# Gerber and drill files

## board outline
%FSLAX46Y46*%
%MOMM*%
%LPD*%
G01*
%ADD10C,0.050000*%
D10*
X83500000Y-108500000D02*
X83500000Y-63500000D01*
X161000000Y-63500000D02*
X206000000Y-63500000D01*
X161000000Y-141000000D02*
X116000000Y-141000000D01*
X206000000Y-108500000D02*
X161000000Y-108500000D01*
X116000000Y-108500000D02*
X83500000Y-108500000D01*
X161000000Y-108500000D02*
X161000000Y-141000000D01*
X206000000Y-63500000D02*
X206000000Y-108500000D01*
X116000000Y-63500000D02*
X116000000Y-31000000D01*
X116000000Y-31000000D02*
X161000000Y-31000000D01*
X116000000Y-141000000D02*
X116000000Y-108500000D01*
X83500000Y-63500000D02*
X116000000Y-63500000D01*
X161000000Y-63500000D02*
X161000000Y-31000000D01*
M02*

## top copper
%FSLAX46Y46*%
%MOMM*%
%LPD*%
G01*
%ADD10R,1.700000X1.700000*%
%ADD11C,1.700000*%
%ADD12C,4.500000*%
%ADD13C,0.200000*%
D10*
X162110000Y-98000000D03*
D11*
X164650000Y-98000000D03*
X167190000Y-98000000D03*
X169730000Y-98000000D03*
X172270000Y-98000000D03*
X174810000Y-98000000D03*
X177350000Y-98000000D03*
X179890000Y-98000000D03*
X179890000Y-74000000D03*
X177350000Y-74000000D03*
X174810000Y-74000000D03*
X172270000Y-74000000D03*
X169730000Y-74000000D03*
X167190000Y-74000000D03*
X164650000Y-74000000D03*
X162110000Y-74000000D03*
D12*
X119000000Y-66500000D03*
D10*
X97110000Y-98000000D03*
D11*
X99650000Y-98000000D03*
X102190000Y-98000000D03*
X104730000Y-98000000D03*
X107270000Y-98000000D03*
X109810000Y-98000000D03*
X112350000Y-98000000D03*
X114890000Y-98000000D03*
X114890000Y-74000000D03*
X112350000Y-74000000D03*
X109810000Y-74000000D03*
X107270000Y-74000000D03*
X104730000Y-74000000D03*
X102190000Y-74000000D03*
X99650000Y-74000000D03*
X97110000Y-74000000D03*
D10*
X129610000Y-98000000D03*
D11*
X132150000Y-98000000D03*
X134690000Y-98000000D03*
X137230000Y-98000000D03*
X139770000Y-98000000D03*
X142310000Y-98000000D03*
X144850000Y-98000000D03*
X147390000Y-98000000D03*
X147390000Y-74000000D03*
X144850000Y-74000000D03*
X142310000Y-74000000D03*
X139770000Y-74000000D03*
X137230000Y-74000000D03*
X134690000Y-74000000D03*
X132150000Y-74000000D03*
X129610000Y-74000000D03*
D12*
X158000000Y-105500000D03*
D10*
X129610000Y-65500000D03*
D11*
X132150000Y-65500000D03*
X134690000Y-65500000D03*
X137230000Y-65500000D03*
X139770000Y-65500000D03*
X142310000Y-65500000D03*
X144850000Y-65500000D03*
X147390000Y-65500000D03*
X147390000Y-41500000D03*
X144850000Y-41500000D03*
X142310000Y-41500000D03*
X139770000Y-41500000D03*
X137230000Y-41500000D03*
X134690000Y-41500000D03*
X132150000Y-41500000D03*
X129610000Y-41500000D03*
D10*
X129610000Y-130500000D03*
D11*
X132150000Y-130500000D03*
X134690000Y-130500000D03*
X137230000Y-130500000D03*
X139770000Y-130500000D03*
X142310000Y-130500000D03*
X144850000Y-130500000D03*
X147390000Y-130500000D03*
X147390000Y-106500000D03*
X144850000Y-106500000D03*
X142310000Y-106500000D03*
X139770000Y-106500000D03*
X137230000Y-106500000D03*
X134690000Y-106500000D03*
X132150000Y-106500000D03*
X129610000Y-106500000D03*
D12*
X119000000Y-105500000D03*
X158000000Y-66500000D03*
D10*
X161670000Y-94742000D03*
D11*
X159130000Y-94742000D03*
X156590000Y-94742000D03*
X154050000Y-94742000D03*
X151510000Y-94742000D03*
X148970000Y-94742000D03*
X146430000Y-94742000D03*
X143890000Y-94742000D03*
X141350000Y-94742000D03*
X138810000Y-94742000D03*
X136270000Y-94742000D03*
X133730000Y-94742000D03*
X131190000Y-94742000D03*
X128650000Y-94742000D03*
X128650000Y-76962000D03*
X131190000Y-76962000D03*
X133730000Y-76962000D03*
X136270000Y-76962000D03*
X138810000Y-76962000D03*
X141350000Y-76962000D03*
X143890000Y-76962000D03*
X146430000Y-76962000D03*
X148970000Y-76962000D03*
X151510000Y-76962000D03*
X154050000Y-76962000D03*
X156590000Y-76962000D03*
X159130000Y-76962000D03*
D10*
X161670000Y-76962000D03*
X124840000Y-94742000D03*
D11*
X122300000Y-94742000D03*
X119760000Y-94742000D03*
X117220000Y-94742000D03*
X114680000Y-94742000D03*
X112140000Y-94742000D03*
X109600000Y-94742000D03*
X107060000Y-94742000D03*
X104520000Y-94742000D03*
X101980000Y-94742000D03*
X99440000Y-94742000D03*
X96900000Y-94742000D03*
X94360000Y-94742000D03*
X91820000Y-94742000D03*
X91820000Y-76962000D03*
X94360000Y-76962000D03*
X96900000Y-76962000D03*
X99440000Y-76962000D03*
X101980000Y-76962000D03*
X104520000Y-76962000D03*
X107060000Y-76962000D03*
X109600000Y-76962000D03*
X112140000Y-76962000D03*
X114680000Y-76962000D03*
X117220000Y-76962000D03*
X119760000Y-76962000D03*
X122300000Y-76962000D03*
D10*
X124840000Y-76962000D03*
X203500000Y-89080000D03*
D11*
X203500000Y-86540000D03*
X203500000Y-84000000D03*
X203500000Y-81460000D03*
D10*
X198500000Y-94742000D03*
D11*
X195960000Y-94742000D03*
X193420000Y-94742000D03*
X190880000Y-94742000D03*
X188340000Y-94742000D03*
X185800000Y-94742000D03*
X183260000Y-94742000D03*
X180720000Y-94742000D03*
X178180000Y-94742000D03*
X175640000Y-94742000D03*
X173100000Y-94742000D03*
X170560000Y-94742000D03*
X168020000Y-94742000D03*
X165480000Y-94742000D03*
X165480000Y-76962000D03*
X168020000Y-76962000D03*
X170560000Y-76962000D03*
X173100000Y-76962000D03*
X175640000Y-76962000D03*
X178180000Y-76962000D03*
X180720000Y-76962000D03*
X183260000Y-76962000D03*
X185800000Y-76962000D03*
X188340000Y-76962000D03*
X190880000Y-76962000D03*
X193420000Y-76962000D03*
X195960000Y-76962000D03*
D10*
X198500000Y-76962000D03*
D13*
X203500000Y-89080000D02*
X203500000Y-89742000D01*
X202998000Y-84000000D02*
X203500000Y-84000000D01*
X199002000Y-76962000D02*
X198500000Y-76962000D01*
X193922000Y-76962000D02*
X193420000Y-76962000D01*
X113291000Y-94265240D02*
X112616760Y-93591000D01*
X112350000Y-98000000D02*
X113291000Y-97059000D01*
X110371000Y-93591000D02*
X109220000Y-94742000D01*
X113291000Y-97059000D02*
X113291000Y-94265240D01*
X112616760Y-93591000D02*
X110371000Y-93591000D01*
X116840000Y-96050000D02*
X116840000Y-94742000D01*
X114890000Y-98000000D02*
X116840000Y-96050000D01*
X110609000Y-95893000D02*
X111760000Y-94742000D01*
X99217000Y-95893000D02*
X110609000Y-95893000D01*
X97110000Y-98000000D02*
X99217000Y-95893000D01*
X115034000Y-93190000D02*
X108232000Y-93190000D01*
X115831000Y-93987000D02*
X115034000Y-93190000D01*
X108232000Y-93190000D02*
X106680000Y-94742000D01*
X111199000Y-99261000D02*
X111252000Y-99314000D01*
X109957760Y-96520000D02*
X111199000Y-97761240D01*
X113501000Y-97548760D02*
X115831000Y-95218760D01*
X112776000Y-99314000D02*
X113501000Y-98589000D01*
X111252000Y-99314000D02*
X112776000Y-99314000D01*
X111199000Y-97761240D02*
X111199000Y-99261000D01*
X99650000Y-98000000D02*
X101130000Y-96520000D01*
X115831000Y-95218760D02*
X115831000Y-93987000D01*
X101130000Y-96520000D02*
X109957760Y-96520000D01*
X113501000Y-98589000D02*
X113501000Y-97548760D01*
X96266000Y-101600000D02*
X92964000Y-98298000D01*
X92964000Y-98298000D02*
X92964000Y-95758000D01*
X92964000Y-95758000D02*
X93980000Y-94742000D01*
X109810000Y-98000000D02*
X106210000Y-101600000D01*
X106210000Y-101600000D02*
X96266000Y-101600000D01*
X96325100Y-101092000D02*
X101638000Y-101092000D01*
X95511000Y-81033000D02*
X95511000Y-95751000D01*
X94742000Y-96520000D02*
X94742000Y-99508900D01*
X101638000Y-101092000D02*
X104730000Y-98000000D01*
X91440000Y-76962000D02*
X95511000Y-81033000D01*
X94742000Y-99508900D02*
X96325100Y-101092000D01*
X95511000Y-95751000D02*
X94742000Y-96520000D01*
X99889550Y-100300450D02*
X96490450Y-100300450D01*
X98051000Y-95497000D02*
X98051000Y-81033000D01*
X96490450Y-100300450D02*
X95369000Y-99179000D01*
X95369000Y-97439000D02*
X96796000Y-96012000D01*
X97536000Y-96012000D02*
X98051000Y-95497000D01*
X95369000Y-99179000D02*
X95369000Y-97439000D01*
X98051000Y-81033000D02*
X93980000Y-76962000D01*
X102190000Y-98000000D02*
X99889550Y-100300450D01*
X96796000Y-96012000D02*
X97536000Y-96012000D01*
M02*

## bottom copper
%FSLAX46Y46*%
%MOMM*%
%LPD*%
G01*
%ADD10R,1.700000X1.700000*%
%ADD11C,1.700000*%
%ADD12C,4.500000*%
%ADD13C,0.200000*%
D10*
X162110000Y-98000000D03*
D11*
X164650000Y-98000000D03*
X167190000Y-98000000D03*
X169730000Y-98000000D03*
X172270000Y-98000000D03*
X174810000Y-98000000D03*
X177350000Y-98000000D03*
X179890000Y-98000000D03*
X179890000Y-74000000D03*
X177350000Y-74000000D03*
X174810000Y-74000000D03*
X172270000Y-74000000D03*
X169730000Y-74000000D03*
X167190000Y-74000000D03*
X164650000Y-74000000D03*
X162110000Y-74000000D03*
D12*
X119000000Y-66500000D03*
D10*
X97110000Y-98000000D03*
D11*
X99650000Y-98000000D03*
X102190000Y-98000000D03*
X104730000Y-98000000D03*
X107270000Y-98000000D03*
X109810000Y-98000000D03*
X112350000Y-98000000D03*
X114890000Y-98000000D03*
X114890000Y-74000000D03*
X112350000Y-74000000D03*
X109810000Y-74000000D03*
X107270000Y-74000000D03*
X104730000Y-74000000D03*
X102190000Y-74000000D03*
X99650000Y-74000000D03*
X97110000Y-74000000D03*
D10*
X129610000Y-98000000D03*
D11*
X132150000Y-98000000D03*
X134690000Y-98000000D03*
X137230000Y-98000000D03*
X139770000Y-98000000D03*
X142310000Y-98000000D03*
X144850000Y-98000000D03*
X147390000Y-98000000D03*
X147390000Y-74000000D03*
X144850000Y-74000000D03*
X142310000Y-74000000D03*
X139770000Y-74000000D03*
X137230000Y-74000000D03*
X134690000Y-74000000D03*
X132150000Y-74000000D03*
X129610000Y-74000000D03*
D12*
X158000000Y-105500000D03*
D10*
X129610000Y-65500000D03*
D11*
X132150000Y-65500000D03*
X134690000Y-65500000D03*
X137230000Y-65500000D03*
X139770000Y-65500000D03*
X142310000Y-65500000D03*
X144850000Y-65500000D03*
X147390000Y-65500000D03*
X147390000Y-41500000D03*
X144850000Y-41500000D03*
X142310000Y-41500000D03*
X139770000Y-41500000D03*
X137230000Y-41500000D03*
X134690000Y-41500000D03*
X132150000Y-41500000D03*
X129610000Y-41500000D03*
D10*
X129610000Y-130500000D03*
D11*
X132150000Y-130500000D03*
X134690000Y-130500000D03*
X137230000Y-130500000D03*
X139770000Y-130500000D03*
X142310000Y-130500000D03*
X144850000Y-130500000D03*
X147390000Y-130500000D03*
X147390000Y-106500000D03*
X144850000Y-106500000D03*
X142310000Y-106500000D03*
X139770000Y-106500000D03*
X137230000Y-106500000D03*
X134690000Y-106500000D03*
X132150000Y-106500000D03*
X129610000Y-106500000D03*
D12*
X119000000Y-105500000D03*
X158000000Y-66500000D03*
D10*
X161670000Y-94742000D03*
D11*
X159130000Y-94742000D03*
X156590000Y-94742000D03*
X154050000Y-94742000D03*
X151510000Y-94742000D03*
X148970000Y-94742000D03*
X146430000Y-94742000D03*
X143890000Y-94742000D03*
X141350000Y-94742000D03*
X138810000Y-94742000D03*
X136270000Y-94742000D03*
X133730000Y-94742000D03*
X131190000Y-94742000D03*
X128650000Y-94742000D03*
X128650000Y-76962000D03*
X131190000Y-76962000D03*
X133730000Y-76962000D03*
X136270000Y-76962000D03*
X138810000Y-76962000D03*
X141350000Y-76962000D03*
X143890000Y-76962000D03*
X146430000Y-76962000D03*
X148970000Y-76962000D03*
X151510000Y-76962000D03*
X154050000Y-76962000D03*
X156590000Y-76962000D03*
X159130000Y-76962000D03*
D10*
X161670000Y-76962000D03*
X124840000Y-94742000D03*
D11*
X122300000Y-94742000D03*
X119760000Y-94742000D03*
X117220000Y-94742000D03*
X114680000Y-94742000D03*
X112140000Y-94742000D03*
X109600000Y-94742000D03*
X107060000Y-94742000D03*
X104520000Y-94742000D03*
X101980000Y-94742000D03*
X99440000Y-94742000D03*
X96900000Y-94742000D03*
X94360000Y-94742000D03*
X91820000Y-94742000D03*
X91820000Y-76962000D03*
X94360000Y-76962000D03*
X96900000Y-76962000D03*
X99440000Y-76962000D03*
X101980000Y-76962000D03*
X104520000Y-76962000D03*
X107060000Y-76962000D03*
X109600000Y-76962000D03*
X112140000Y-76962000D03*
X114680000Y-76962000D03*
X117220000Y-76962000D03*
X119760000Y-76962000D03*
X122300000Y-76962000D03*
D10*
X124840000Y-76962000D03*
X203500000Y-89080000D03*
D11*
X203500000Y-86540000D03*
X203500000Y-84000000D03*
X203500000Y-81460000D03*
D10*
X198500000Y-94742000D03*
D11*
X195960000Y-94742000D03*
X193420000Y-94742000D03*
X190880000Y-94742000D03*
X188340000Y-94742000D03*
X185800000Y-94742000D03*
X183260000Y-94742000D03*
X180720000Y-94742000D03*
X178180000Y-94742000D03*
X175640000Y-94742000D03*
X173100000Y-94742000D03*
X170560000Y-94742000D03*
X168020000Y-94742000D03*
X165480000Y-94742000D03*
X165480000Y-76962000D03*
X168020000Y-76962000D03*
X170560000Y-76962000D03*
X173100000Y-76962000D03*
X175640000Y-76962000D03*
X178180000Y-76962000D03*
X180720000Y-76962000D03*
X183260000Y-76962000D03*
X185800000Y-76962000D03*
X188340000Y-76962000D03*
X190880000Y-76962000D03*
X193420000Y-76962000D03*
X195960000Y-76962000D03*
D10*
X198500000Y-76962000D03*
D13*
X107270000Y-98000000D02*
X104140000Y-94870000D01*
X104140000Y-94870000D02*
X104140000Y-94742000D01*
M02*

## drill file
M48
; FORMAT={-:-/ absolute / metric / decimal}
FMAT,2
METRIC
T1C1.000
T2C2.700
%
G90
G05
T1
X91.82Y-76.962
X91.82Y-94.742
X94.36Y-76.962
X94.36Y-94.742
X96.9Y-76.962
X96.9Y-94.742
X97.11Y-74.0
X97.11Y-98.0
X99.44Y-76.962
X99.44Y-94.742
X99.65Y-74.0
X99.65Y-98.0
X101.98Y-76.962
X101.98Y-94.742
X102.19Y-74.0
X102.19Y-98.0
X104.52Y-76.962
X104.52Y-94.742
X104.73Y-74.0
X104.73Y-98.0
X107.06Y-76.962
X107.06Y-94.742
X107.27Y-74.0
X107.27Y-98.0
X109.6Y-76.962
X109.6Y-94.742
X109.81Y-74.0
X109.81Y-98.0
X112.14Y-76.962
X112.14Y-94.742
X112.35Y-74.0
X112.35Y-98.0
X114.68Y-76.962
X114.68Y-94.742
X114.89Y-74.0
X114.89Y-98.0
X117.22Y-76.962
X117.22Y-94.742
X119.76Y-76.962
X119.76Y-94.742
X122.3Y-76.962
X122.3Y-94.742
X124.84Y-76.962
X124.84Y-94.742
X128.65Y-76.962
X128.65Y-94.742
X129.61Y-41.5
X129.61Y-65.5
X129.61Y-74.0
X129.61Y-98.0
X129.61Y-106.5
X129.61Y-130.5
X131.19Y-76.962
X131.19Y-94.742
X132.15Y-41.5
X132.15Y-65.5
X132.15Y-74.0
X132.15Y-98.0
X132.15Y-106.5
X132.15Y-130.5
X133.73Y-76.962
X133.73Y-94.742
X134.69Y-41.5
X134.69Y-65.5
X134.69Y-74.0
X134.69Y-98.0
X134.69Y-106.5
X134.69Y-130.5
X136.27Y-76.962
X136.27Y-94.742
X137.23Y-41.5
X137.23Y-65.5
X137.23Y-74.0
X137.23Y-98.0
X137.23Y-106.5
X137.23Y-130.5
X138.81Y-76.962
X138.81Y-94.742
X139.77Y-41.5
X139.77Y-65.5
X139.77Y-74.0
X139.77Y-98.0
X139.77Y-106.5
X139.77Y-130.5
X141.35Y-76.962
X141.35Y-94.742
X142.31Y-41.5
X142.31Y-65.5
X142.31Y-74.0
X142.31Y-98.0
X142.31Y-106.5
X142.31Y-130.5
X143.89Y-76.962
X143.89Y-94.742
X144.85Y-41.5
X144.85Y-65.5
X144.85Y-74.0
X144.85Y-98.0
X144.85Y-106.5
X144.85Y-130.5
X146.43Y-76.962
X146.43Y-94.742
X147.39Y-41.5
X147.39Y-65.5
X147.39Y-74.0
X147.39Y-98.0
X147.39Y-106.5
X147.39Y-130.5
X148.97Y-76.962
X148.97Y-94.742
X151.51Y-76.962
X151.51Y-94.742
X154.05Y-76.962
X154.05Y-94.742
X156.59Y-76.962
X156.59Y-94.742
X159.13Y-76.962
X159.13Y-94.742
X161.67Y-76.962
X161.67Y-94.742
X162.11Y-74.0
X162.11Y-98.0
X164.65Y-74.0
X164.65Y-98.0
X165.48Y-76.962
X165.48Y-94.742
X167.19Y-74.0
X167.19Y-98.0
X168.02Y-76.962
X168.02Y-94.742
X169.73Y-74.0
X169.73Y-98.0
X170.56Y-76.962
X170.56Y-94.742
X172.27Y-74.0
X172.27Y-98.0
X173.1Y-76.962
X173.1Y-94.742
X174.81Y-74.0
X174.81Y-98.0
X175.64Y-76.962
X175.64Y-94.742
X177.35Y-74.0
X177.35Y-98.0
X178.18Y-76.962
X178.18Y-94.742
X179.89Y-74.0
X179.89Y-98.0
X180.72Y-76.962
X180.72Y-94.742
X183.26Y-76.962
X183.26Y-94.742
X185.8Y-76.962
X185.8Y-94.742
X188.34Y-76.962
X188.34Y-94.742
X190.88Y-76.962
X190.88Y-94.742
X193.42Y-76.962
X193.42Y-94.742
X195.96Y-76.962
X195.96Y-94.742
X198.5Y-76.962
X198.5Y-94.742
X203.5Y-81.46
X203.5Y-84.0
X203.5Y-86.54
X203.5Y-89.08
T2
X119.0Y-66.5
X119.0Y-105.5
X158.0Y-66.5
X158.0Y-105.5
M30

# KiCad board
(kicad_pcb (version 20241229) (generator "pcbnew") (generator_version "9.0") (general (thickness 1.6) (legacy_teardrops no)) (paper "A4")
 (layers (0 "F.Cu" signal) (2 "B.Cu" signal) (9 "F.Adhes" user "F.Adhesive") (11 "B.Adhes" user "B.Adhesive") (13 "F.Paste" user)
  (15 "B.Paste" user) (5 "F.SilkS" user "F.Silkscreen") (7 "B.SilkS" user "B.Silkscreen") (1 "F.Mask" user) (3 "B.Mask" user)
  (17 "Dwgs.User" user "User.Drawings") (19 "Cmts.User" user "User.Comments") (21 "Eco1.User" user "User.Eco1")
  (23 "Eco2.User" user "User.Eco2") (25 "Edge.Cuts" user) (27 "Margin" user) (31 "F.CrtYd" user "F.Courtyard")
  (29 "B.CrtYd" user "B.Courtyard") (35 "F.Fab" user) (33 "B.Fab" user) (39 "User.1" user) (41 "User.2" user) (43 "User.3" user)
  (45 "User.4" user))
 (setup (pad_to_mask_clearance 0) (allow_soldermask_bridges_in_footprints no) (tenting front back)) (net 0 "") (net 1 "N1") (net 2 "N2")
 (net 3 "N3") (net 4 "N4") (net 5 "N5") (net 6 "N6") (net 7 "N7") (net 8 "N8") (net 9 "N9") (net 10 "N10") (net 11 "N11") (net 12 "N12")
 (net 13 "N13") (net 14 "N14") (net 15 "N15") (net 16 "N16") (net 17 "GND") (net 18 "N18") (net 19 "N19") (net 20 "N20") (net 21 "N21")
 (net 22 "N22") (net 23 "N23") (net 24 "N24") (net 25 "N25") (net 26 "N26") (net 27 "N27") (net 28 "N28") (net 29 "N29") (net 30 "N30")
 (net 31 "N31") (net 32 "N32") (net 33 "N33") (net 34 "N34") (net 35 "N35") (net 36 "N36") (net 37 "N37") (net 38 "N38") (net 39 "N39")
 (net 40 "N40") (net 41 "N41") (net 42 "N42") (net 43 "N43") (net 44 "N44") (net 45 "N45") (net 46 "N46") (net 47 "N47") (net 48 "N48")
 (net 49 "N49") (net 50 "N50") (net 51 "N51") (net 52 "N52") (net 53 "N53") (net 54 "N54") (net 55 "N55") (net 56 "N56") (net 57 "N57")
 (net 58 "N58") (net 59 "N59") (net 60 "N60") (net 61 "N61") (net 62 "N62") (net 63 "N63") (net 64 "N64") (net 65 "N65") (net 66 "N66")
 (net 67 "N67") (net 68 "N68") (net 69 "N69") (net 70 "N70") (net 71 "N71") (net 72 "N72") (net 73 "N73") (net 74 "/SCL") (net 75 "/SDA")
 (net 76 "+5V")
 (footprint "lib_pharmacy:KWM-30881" (layer "F.Cu") (at 171 86)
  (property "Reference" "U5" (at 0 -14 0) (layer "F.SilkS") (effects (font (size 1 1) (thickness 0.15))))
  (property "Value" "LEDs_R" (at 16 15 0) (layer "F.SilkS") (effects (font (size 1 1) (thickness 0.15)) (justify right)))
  (pad "1" thru_hole rect (at -8.89 12 90) (size 1.7 1.7) (drill 1) (layers "*.Cu" "*.Mask") (remove_unused_layers no) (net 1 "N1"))
  (pad "2" thru_hole circle (at -6.35 12 90) (size 1.7 1.7) (drill 1) (layers "*.Cu" "*.Mask") (remove_unused_layers no) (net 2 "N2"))
  (pad "3" thru_hole circle (at -3.81 12 90) (size 1.7 1.7) (drill 1) (layers "*.Cu" "*.Mask") (remove_unused_layers no) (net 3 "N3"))
  (pad "4" thru_hole circle (at -1.27 12 90) (size 1.7 1.7) (drill 1) (layers "*.Cu" "*.Mask") (remove_unused_layers no) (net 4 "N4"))
  (pad "5" thru_hole circle (at 1.27 12 90) (size 1.7 1.7) (drill 1) (layers "*.Cu" "*.Mask") (remove_unused_layers no) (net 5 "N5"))
  (pad "6" thru_hole circle (at 3.81 12 90) (size 1.7 1.7) (drill 1) (layers "*.Cu" "*.Mask") (remove_unused_layers no) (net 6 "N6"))
  (pad "7" thru_hole circle (at 6.35 12 90) (size 1.7 1.7) (drill 1) (layers "*.Cu" "*.Mask") (remove_unused_layers no) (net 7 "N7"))
  (pad "8" thru_hole circle (at 8.89 12 90) (size 1.7 1.7) (drill 1) (layers "*.Cu" "*.Mask") (remove_unused_layers no) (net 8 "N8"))
  (pad "9" thru_hole circle (at 8.89 -12 90) (size 1.7 1.7) (drill 1) (layers "*.Cu" "*.Mask") (remove_unused_layers no) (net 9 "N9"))
  (pad "10" thru_hole circle (at 6.35 -12 90) (size 1.7 1.7) (drill 1) (layers "*.Cu" "*.Mask") (remove_unused_layers no) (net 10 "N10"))
  (pad "11" thru_hole circle (at 3.81 -12 90) (size 1.7 1.7) (drill 1) (layers "*.Cu" "*.Mask") (remove_unused_layers no) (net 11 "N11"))
  (pad "12" thru_hole circle (at 1.27 -12 90) (size 1.7 1.7) (drill 1) (layers "*.Cu" "*.Mask") (remove_unused_layers no) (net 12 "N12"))
  (pad "13" thru_hole circle (at -1.27 -12 90) (size 1.7 1.7) (drill 1) (layers "*.Cu" "*.Mask") (remove_unused_layers no) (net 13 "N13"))
  (pad "14" thru_hole circle (at -3.81 -12 90) (size 1.7 1.7) (drill 1) (layers "*.Cu" "*.Mask") (remove_unused_layers no) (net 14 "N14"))
  (pad "15" thru_hole circle (at -6.35 -12 90) (size 1.7 1.7) (drill 1) (layers "*.Cu" "*.Mask") (remove_unused_layers no) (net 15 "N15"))
  (pad "16" thru_hole circle (at -8.89 -12 90) (size 1.7 1.7) (drill 1) (layers "*.Cu" "*.Mask") (remove_unused_layers no) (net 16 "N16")))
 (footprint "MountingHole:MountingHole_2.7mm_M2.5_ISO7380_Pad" (layer "F.Cu") (at 119 66.5)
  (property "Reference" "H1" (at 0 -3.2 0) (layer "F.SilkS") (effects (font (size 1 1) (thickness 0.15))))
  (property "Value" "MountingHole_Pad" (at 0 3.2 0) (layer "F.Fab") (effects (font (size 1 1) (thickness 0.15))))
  (pad "1" thru_hole circle (at 0 0) (size 4.5 4.5) (drill 2.7) (layers "*.Cu" "*.Mask") (remove_unused_layers no) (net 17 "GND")
   (zone_connect 2)))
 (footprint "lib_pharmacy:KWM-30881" (layer "F.Cu") (at 106 86)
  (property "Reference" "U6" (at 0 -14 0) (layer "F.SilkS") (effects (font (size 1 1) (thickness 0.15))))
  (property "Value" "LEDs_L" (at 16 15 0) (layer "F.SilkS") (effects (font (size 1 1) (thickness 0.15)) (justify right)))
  (pad "1" thru_hole rect (at -8.89 12 90) (size 1.7 1.7) (drill 1) (layers "*.Cu" "*.Mask") (remove_unused_layers no) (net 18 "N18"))
  (pad "2" thru_hole circle (at -6.35 12 90) (size 1.7 1.7) (drill 1) (layers "*.Cu" "*.Mask") (remove_unused_layers no) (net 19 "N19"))
  (pad "3" thru_hole circle (at -3.81 12 90) (size 1.7 1.7) (drill 1) (layers "*.Cu" "*.Mask") (remove_unused_layers no) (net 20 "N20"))
  (pad "4" thru_hole circle (at -1.27 12 90) (size 1.7 1.7) (drill 1) (layers "*.Cu" "*.Mask") (remove_unused_layers no) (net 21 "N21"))
  (pad "5" thru_hole circle (at 1.27 12 90) (size 1.7 1.7) (drill 1) (layers "*.Cu" "*.Mask") (remove_unused_layers no) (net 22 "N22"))
  (pad "6" thru_hole circle (at 3.81 12 90) (size 1.7 1.7) (drill 1) (layers "*.Cu" "*.Mask") (remove_unused_layers no) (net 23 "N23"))
  (pad "7" thru_hole circle (at 6.35 12 90) (size 1.7 1.7) (drill 1) (layers "*.Cu" "*.Mask") (remove_unused_layers no) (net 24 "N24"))
  (pad "8" thru_hole circle (at 8.89 12 90) (size 1.7 1.7) (drill 1) (layers "*.Cu" "*.Mask") (remove_unused_layers no) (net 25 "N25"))
  (pad "9" thru_hole circle (at 8.89 -12 90) (size 1.7 1.7) (drill 1) (layers "*.Cu" "*.Mask") (remove_unused_layers no) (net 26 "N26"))
  (pad "10" thru_hole circle (at 6.35 -12 90) (size 1.7 1.7) (drill 1) (layers "*.Cu" "*.Mask") (remove_unused_layers no) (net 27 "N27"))
  (pad "11" thru_hole circle (at 3.81 -12 90) (size 1.7 1.7) (drill 1) (layers "*.Cu" "*.Mask") (remove_unused_layers no) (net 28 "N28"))
  (pad "12" thru_hole circle (at 1.27 -12 90) (size 1.7 1.7) (drill 1) (layers "*.Cu" "*.Mask") (remove_unused_layers no) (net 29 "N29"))
  (pad "13" thru_hole circle (at -1.27 -12 90) (size 1.7 1.7) (drill 1) (layers "*.Cu" "*.Mask") (remove_unused_layers no) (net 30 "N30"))
  (pad "14" thru_hole circle (at -3.81 -12 90) (size 1.7 1.7) (drill 1) (layers "*.Cu" "*.Mask") (remove_unused_layers no) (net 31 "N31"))
  (pad "15" thru_hole circle (at -6.35 -12 90) (size 1.7 1.7) (drill 1) (layers "*.Cu" "*.Mask") (remove_unused_layers no) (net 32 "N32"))
  (pad "16" thru_hole circle (at -8.89 -12 90) (size 1.7 1.7) (drill 1) (layers "*.Cu" "*.Mask") (remove_unused_layers no) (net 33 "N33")))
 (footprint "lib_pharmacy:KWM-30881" (layer "F.Cu") (at 138.5 86)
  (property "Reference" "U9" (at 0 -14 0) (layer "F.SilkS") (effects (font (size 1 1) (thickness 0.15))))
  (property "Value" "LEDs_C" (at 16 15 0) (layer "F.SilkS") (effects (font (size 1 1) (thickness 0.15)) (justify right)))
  (pad "1" thru_hole rect (at -8.89 12 90) (size 1.7 1.7) (drill 1) (layers "*.Cu" "*.Mask") (remove_unused_layers no) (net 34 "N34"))
  (pad "2" thru_hole circle (at -6.35 12 90) (size 1.7 1.7) (drill 1) (layers "*.Cu" "*.Mask") (remove_unused_layers no) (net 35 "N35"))
  (pad "3" thru_hole circle (at -3.81 12 90) (size 1.7 1.7) (drill 1) (layers "*.Cu" "*.Mask") (remove_unused_layers no) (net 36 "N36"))
  (pad "4" thru_hole circle (at -1.27 12 90) (size 1.7 1.7) (drill 1) (layers "*.Cu" "*.Mask") (remove_unused_layers no) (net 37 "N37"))
  (pad "5" thru_hole circle (at 1.27 12 90) (size 1.7 1.7) (drill 1) (layers "*.Cu" "*.Mask") (remove_unused_layers no) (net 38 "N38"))
  (pad "6" thru_hole circle (at 3.81 12 90) (size 1.7 1.7) (drill 1) (layers "*.Cu" "*.Mask") (remove_unused_layers no) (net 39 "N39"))
  (pad "7" thru_hole circle (at 6.35 12 90) (size 1.7 1.7) (drill 1) (layers "*.Cu" "*.Mask") (remove_unused_layers no) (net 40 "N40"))
  (pad "8" thru_hole circle (at 8.89 12 90) (size 1.7 1.7) (drill 1) (layers "*.Cu" "*.Mask") (remove_unused_layers no) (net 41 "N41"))
  (pad "9" thru_hole circle (at 8.89 -12 90) (size 1.7 1.7) (drill 1) (layers "*.Cu" "*.Mask") (remove_unused_layers no) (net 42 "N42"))
  (pad "10" thru_hole circle (at 6.35 -12 90) (size 1.7 1.7) (drill 1) (layers "*.Cu" "*.Mask") (remove_unused_layers no) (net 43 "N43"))
  (pad "11" thru_hole circle (at 3.81 -12 90) (size 1.7 1.7) (drill 1) (layers "*.Cu" "*.Mask") (remove_unused_layers no) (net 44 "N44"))
  (pad "12" thru_hole circle (at 1.27 -12 90) (size 1.7 1.7) (drill 1) (layers "*.Cu" "*.Mask") (remove_unused_layers no) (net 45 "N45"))
  (pad "13" thru_hole circle (at -1.27 -12 90) (size 1.7 1.7) (drill 1) (layers "*.Cu" "*.Mask") (remove_unused_layers no) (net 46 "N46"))
  (pad "14" thru_hole circle (at -3.81 -12 90) (size 1.7 1.7) (drill 1) (layers "*.Cu" "*.Mask") (remove_unused_layers no) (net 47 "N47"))
  (pad "15" thru_hole circle (at -6.35 -12 90) (size 1.7 1.7) (drill 1) (layers "*.Cu" "*.Mask") (remove_unused_layers no) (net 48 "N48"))
  (pad "16" thru_hole circle (at -8.89 -12 90) (size 1.7 1.7) (drill 1) (layers "*.Cu" "*.Mask") (remove_unused_layers no) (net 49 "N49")))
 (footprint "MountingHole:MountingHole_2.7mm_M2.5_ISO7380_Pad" (layer "F.Cu") (at 158 105.5)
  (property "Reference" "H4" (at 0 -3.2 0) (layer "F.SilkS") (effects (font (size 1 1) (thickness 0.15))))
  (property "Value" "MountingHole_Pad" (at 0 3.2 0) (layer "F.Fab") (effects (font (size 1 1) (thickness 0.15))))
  (pad "1" thru_hole circle (at 0 0) (size 4.5 4.5) (drill 2.7) (layers "*.Cu" "*.Mask") (remove_unused_layers no) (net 17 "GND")
   (zone_connect 2)))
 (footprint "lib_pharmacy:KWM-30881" (layer "F.Cu") (at 138.5 53.5)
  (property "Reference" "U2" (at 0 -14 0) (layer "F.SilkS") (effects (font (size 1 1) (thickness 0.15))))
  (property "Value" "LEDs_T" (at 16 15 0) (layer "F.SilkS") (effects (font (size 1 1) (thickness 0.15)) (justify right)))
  (pad "1" thru_hole rect (at -8.89 12 90) (size 1.7 1.7) (drill 1) (layers "*.Cu" "*.Mask") (remove_unused_layers no) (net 18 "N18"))
  (pad "2" thru_hole circle (at -6.35 12 90) (size 1.7 1.7) (drill 1) (layers "*.Cu" "*.Mask") (remove_unused_layers no) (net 19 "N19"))
  (pad "3" thru_hole circle (at -3.81 12 90) (size 1.7 1.7) (drill 1) (layers "*.Cu" "*.Mask") (remove_unused_layers no) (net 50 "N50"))
  (pad "4" thru_hole circle (at -1.27 12 90) (size 1.7 1.7) (drill 1) (layers "*.Cu" "*.Mask") (remove_unused_layers no) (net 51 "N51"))
  (pad "5" thru_hole circle (at 1.27 12 90) (size 1.7 1.7) (drill 1) (layers "*.Cu" "*.Mask") (remove_unused_layers no) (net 22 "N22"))
  (pad "6" thru_hole circle (at 3.81 12 90) (size 1.7 1.7) (drill 1) (layers "*.Cu" "*.Mask") (remove_unused_layers no) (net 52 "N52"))
  (pad "7" thru_hole circle (at 6.35 12 90) (size 1.7 1.7) (drill 1) (layers "*.Cu" "*.Mask") (remove_unused_layers no) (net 24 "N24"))
  (pad "8" thru_hole circle (at 8.89 12 90) (size 1.7 1.7) (drill 1) (layers "*.Cu" "*.Mask") (remove_unused_layers no) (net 25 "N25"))
  (pad "9" thru_hole circle (at 8.89 -12 90) (size 1.7 1.7) (drill 1) (layers "*.Cu" "*.Mask") (remove_unused_layers no) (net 26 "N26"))
  (pad "10" thru_hole circle (at 6.35 -12 90) (size 1.7 1.7) (drill 1) (layers "*.Cu" "*.Mask") (remove_unused_layers no) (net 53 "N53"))
  (pad "11" thru_hole circle (at 3.81 -12 90) (size 1.7 1.7) (drill 1) (layers "*.Cu" "*.Mask") (remove_unused_layers no) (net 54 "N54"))
  (pad "12" thru_hole circle (at 1.27 -12 90) (size 1.7 1.7) (drill 1) (layers "*.Cu" "*.Mask") (remove_unused_layers no) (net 29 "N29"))
  (pad "13" thru_hole circle (at -1.27 -12 90) (size 1.7 1.7) (drill 1) (layers "*.Cu" "*.Mask") (remove_unused_layers no) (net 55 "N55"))
  (pad "14" thru_hole circle (at -3.81 -12 90) (size 1.7 1.7) (drill 1) (layers "*.Cu" "*.Mask") (remove_unused_layers no) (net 31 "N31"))
  (pad "15" thru_hole circle (at -6.35 -12 90) (size 1.7 1.7) (drill 1) (layers "*.Cu" "*.Mask") (remove_unused_layers no) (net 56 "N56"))
  (pad "16" thru_hole circle (at -8.89 -12 90) (size 1.7 1.7) (drill 1) (layers "*.Cu" "*.Mask") (remove_unused_layers no) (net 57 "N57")))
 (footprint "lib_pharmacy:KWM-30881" (layer "F.Cu") (at 138.5 118.5)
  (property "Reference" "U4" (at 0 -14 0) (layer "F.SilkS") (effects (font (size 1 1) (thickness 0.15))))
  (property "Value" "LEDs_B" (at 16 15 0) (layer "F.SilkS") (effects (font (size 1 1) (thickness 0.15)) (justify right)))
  (pad "1" thru_hole rect (at -8.89 12 90) (size 1.7 1.7) (drill 1) (layers "*.Cu" "*.Mask") (remove_unused_layers no) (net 1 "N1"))
  (pad "2" thru_hole circle (at -6.35 12 90) (size 1.7 1.7) (drill 1) (layers "*.Cu" "*.Mask") (remove_unused_layers no) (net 2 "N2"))
  (pad "3" thru_hole circle (at -3.81 12 90) (size 1.7 1.7) (drill 1) (layers "*.Cu" "*.Mask") (remove_unused_layers no) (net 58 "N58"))
  (pad "4" thru_hole circle (at -1.27 12 90) (size 1.7 1.7) (drill 1) (layers "*.Cu" "*.Mask") (remove_unused_layers no) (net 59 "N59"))
  (pad "5" thru_hole circle (at 1.27 12 90) (size 1.7 1.7) (drill 1) (layers "*.Cu" "*.Mask") (remove_unused_layers no) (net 5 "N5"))
  (pad "6" thru_hole circle (at 3.81 12 90) (size 1.7 1.7) (drill 1) (layers "*.Cu" "*.Mask") (remove_unused_layers no) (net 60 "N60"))
  (pad "7" thru_hole circle (at 6.35 12 90) (size 1.7 1.7) (drill 1) (layers "*.Cu" "*.Mask") (remove_unused_layers no) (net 7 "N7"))
  (pad "8" thru_hole circle (at 8.89 12 90) (size 1.7 1.7) (drill 1) (layers "*.Cu" "*.Mask") (remove_unused_layers no) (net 8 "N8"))
  (pad "9" thru_hole circle (at 8.89 -12 90) (size 1.7 1.7) (drill 1) (layers "*.Cu" "*.Mask") (remove_unused_layers no) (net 9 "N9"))
  (pad "10" thru_hole circle (at 6.35 -12 90) (size 1.7 1.7) (drill 1) (layers "*.Cu" "*.Mask") (remove_unused_layers no) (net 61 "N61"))
  (pad "11" thru_hole circle (at 3.81 -12 90) (size 1.7 1.7) (drill 1) (layers "*.Cu" "*.Mask") (remove_unused_layers no) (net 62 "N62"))
  (pad "12" thru_hole circle (at 1.27 -12 90) (size 1.7 1.7) (drill 1) (layers "*.Cu" "*.Mask") (remove_unused_layers no) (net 12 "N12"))
  (pad "13" thru_hole circle (at -1.27 -12 90) (size 1.7 1.7) (drill 1) (layers "*.Cu" "*.Mask") (remove_unused_layers no) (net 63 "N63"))
  (pad "14" thru_hole circle (at -3.81 -12 90) (size 1.7 1.7) (drill 1) (layers "*.Cu" "*.Mask") (remove_unused_layers no) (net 14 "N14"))
  (pad "15" thru_hole circle (at -6.35 -12 90) (size 1.7 1.7) (drill 1) (layers "*.Cu" "*.Mask") (remove_unused_layers no) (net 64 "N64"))
  (pad "16" thru_hole circle (at -8.89 -12 90) (size 1.7 1.7) (drill 1) (layers "*.Cu" "*.Mask") (remove_unused_layers no) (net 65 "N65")))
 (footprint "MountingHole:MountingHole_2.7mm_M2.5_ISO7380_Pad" (layer "F.Cu") (at 119 105.5)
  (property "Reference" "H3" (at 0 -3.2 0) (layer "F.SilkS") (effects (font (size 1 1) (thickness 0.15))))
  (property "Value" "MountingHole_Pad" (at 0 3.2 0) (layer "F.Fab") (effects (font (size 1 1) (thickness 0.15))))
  (pad "1" thru_hole circle (at 0 0) (size 4.5 4.5) (drill 2.7) (layers "*.Cu" "*.Mask") (remove_unused_layers no) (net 17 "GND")
   (zone_connect 2)))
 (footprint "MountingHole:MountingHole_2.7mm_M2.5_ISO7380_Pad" (layer "F.Cu") (at 158 66.5)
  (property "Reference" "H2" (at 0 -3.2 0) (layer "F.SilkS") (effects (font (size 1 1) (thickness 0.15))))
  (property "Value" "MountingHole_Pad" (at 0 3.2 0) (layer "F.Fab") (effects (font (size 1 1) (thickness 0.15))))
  (pad "1" thru_hole circle (at 0 0) (size 4.5 4.5) (drill 2.7) (layers "*.Cu" "*.Mask") (remove_unused_layers no) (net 17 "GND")
   (zone_connect 2)))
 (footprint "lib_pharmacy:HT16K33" (layer "B.Cu") (at 161.67 94.742 180)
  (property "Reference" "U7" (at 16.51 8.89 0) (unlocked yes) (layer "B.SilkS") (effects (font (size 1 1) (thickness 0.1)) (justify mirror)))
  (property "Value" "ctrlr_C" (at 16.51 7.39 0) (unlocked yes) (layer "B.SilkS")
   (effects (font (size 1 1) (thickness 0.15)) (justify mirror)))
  (pad "1" thru_hole rect (at 0 0 90) (size 1.7 1.7) (drill 1) (layers "*.Cu" "*.Mask") (remove_unused_layers no) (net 17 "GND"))
  (pad "2" thru_hole circle (at 2.54 0 90) (size 1.7 1.7) (drill 1) (layers "*.Cu" "*.Mask") (remove_unused_layers no) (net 42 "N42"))
  (pad "3" thru_hole circle (at 5.08 0 90) (size 1.7 1.7) (drill 1) (layers "*.Cu" "*.Mask") (remove_unused_layers no) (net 47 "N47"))
  (pad "4" thru_hole circle (at 7.62 0 90) (size 1.7 1.7) (drill 1) (layers "*.Cu" "*.Mask") (remove_unused_layers no) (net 41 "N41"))
  (pad "5" thru_hole circle (at 10.16 0 90) (size 1.7 1.7) (drill 1) (layers "*.Cu" "*.Mask") (remove_unused_layers no) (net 45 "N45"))
  (pad "6" thru_hole circle (at 12.7 0 90) (size 1.7 1.7) (drill 1) (layers "*.Cu" "*.Mask") (remove_unused_layers no) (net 34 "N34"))
  (pad "7" thru_hole circle (at 15.24 0 90) (size 1.7 1.7) (drill 1) (layers "*.Cu" "*.Mask") (remove_unused_layers no) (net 40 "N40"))
  (pad "8" thru_hole circle (at 17.78 0 90) (size 1.7 1.7) (drill 1) (layers "*.Cu" "*.Mask") (remove_unused_layers no) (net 35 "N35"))
  (pad "9" thru_hole circle (at 20.32 0 90) (size 1.7 1.7) (drill 1) (layers "*.Cu" "*.Mask") (remove_unused_layers no) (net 38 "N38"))
  (pad "10" thru_hole circle (at 22.86 0 90) (size 1.7 1.7) (drill 1) (layers "*.Cu" "*.Mask") (remove_unused_layers no) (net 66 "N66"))
  (pad "11" thru_hole circle (at 25.4 0 90) (size 1.7 1.7) (drill 1) (layers "*.Cu" "*.Mask") (remove_unused_layers no) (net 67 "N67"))
  (pad "12" thru_hole circle (at 27.94 0 90) (size 1.7 1.7) (drill 1) (layers "*.Cu" "*.Mask") (remove_unused_layers no) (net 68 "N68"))
  (pad "13" thru_hole circle (at 30.48 0 90) (size 1.7 1.7) (drill 1) (layers "*.Cu" "*.Mask") (remove_unused_layers no) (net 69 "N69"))
  (pad "14" thru_hole circle (at 33.02 0 90) (size 1.7 1.7) (drill 1) (layers "*.Cu" "*.Mask") (remove_unused_layers no) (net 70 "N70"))
  (pad "15" thru_hole circle (at 33.02 17.78 90) (size 1.7 1.7) (drill 1) (layers "*.Cu" "*.Mask") (remove_unused_layers no) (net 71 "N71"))
  (pad "16" thru_hole circle (at 30.48 17.78 90) (size 1.7 1.7) (drill 1) (layers "*.Cu" "*.Mask") (remove_unused_layers no) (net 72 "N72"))
  (pad "17" thru_hole circle (at 27.94 17.78 90) (size 1.7 1.7) (drill 1) (layers "*.Cu" "*.Mask") (remove_unused_layers no) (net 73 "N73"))
  (pad "18" thru_hole circle (at 25.4 17.78 90) (size 1.7 1.7) (drill 1) (layers "*.Cu" "*.Mask") (remove_unused_layers no) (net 49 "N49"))
  (pad "19" thru_hole circle (at 22.86 17.78 90) (size 1.7 1.7) (drill 1) (layers "*.Cu" "*.Mask") (remove_unused_layers no) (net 48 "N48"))
  (pad "20" thru_hole circle (at 20.32 17.78 90) (size 1.7 1.7) (drill 1) (layers "*.Cu" "*.Mask") (remove_unused_layers no) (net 44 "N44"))
  (pad "21" thru_hole circle (at 17.78 17.78 90) (size 1.7 1.7) (drill 1) (layers "*.Cu" "*.Mask") (remove_unused_layers no) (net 39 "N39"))
  (pad "22" thru_hole circle (at 15.24 17.78 90) (size 1.7 1.7) (drill 1) (layers "*.Cu" "*.Mask") (remove_unused_layers no) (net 43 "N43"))
  (pad "23" thru_hole circle (at 12.7 17.78 90) (size 1.7 1.7) (drill 1) (layers "*.Cu" "*.Mask") (remove_unused_layers no) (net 37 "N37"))
  (pad "24" thru_hole circle (at 10.16 17.78 90) (size 1.7 1.7) (drill 1) (layers "*.Cu" "*.Mask") (remove_unused_layers no) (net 36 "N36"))
  (pad "25" thru_hole circle (at 7.62 17.78 90) (size 1.7 1.7) (drill 1) (layers "*.Cu" "*.Mask") (remove_unused_layers no) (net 46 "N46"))
  (pad "26" thru_hole circle (at 5.08 17.78 90) (size 1.7 1.7) (drill 1) (layers "*.Cu" "*.Mask") (remove_unused_layers no) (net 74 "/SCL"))
  (pad "27" thru_hole circle (at 2.54 17.78 90) (size 1.7 1.7) (drill 1) (layers "*.Cu" "*.Mask") (remove_unused_layers no) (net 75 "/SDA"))
  (pad "28" thru_hole rect (at 0 17.78 90) (size 1.7 1.7) (drill 1) (layers "*.Cu" "*.Mask") (remove_unused_layers no) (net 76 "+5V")))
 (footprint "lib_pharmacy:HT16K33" (layer "B.Cu") (at 124.84 94.742 180)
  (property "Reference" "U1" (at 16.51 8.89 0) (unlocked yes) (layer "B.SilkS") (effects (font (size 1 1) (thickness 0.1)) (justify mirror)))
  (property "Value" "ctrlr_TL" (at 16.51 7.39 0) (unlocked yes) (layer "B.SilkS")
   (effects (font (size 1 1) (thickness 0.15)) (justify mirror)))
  (pad "1" thru_hole rect (at 0 0 90) (size 1.7 1.7) (drill 1) (layers "*.Cu" "*.Mask") (remove_unused_layers no) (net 17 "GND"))
  (pad "2" thru_hole circle (at 2.54 0 90) (size 1.7 1.7) (drill 1) (layers "*.Cu" "*.Mask") (remove_unused_layers no) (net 26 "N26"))
  (pad "3" thru_hole circle (at 5.08 0 90) (size 1.7 1.7) (drill 1) (layers "*.Cu" "*.Mask") (remove_unused_layers no) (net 31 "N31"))
  (pad "4" thru_hole circle (at 7.62 0 90) (size 1.7 1.7) (drill 1) (layers "*.Cu" "*.Mask") (remove_unused_layers no) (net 25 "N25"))
  (pad "5" thru_hole circle (at 10.16 0 90) (size 1.7 1.7) (drill 1) (layers "*.Cu" "*.Mask") (remove_unused_layers no) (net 29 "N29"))
  (pad "6" thru_hole circle (at 12.7 0 90) (size 1.7 1.7) (drill 1) (layers "*.Cu" "*.Mask") (remove_unused_layers no) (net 18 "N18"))
  (pad "7" thru_hole circle (at 15.24 0 90) (size 1.7 1.7) (drill 1) (layers "*.Cu" "*.Mask") (remove_unused_layers no) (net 24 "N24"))
  (pad "8" thru_hole circle (at 17.78 0 90) (size 1.7 1.7) (drill 1) (layers "*.Cu" "*.Mask") (remove_unused_layers no) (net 19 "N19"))
  (pad "9" thru_hole circle (at 20.32 0 90) (size 1.7 1.7) (drill 1) (layers "*.Cu" "*.Mask") (remove_unused_layers no) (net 22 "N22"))
  (pad "10" thru_hole circle (at 22.86 0 90) (size 1.7 1.7) (drill 1) (layers "*.Cu" "*.Mask") (remove_unused_layers no) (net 33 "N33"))
  (pad "11" thru_hole circle (at 25.4 0 90) (size 1.7 1.7) (drill 1) (layers "*.Cu" "*.Mask") (remove_unused_layers no) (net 32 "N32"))
  (pad "12" thru_hole circle (at 27.94 0 90) (size 1.7 1.7) (drill 1) (layers "*.Cu" "*.Mask") (remove_unused_layers no) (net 28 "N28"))
  (pad "13" thru_hole circle (at 30.48 0 90) (size 1.7 1.7) (drill 1) (layers "*.Cu" "*.Mask") (remove_unused_layers no) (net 23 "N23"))
  (pad "14" thru_hole circle (at 33.02 0 90) (size 1.7 1.7) (drill 1) (layers "*.Cu" "*.Mask") (remove_unused_layers no) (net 27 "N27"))
  (pad "15" thru_hole circle (at 33.02 17.78 90) (size 1.7 1.7) (drill 1) (layers "*.Cu" "*.Mask") (remove_unused_layers no) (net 21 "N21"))
  (pad "16" thru_hole circle (at 30.48 17.78 90) (size 1.7 1.7) (drill 1) (layers "*.Cu" "*.Mask") (remove_unused_layers no) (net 20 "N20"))
  (pad "17" thru_hole circle (at 27.94 17.78 90) (size 1.7 1.7) (drill 1) (layers "*.Cu" "*.Mask") (remove_unused_layers no) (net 30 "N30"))
  (pad "18" thru_hole circle (at 25.4 17.78 90) (size 1.7 1.7) (drill 1) (layers "*.Cu" "*.Mask") (remove_unused_layers no) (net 57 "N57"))
  (pad "19" thru_hole circle (at 22.86 17.78 90) (size 1.7 1.7) (drill 1) (layers "*.Cu" "*.Mask") (remove_unused_layers no) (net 56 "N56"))
  (pad "20" thru_hole circle (at 20.32 17.78 90) (size 1.7 1.7) (drill 1) (layers "*.Cu" "*.Mask") (remove_unused_layers no) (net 54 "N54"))
  (pad "21" thru_hole circle (at 17.78 17.78 90) (size 1.7 1.7) (drill 1) (layers "*.Cu" "*.Mask") (remove_unused_layers no) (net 52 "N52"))
  (pad "22" thru_hole circle (at 15.24 17.78 90) (size 1.7 1.7) (drill 1) (layers "*.Cu" "*.Mask") (remove_unused_layers no) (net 53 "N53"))
  (pad "23" thru_hole circle (at 12.7 17.78 90) (size 1.7 1.7) (drill 1) (layers "*.Cu" "*.Mask") (remove_unused_layers no) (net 51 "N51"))
  (pad "24" thru_hole circle (at 10.16 17.78 90) (size 1.7 1.7) (drill 1) (layers "*.Cu" "*.Mask") (remove_unused_layers no) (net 50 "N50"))
  (pad "25" thru_hole circle (at 7.62 17.78 90) (size 1.7 1.7) (drill 1) (layers "*.Cu" "*.Mask") (remove_unused_layers no) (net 55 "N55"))
  (pad "26" thru_hole circle (at 5.08 17.78 90) (size 1.7 1.7) (drill 1) (layers "*.Cu" "*.Mask") (remove_unused_layers no) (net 74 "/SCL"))
  (pad "27" thru_hole circle (at 2.54 17.78 90) (size 1.7 1.7) (drill 1) (layers "*.Cu" "*.Mask") (remove_unused_layers no) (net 75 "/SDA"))
  (pad "28" thru_hole rect (at 0 17.78 90) (size 1.7 1.7) (drill 1) (layers "*.Cu" "*.Mask") (remove_unused_layers no) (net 76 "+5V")))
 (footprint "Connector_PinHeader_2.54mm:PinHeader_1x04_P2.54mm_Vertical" (layer "B.Cu") (at 203.5 89.08)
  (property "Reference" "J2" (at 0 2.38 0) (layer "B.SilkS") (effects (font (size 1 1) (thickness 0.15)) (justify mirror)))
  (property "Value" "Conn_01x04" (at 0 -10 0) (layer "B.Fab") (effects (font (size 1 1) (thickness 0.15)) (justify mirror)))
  (pad "1" thru_hole rect (at 0 0) (size 1.7 1.7) (drill 1) (layers "*.Cu" "*.Mask") (remove_unused_layers no) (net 17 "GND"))
  (pad "2" thru_hole circle (at 0 -2.54) (size 1.7 1.7) (drill 1) (layers "*.Cu" "*.Mask") (remove_unused_layers no) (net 74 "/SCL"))
  (pad "3" thru_hole circle (at 0 -5.08) (size 1.7 1.7) (drill 1) (layers "*.Cu" "*.Mask") (remove_unused_layers no) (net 75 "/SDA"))
  (pad "4" thru_hole circle (at 0 -7.62) (size 1.7 1.7) (drill 1) (layers "*.Cu" "*.Mask") (remove_unused_layers no) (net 76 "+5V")))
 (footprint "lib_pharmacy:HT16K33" (layer "B.Cu") (at 198.5 94.742 180)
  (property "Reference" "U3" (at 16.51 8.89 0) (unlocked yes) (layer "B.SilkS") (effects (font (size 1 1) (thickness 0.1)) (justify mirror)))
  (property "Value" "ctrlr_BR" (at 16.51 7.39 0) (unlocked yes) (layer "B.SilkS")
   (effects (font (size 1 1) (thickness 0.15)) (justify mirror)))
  (pad "1" thru_hole rect (at 0 0 90) (size 1.7 1.7) (drill 1) (layers "*.Cu" "*.Mask") (remove_unused_layers no) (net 17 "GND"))
  (pad "2" thru_hole circle (at 2.54 0 90) (size 1.7 1.7) (drill 1) (layers "*.Cu" "*.Mask") (remove_unused_layers no) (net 9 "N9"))
  (pad "3" thru_hole circle (at 5.08 0 90) (size 1.7 1.7) (drill 1) (layers "*.Cu" "*.Mask") (remove_unused_layers no) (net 14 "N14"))
  (pad "4" thru_hole circle (at 7.62 0 90) (size 1.7 1.7) (drill 1) (layers "*.Cu" "*.Mask") (remove_unused_layers no) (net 8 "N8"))
  (pad "5" thru_hole circle (at 10.16 0 90) (size 1.7 1.7) (drill 1) (layers "*.Cu" "*.Mask") (remove_unused_layers no) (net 12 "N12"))
  (pad "6" thru_hole circle (at 12.7 0 90) (size 1.7 1.7) (drill 1) (layers "*.Cu" "*.Mask") (remove_unused_layers no) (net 1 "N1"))
  (pad "7" thru_hole circle (at 15.24 0 90) (size 1.7 1.7) (drill 1) (layers "*.Cu" "*.Mask") (remove_unused_layers no) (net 7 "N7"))
  (pad "8" thru_hole circle (at 17.78 0 90) (size 1.7 1.7) (drill 1) (layers "*.Cu" "*.Mask") (remove_unused_layers no) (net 2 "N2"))
  (pad "9" thru_hole circle (at 20.32 0 90) (size 1.7 1.7) (drill 1) (layers "*.Cu" "*.Mask") (remove_unused_layers no) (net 5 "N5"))
  (pad "10" thru_hole circle (at 22.86 0 90) (size 1.7 1.7) (drill 1) (layers "*.Cu" "*.Mask") (remove_unused_layers no) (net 65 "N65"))
  (pad "11" thru_hole circle (at 25.4 0 90) (size 1.7 1.7) (drill 1) (layers "*.Cu" "*.Mask") (remove_unused_layers no) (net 64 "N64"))
  (pad "12" thru_hole circle (at 27.94 0 90) (size 1.7 1.7) (drill 1) (layers "*.Cu" "*.Mask") (remove_unused_layers no) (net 62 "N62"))
  (pad "13" thru_hole circle (at 30.48 0 90) (size 1.7 1.7) (drill 1) (layers "*.Cu" "*.Mask") (remove_unused_layers no) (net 60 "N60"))
  (pad "14" thru_hole circle (at 33.02 0 90) (size 1.7 1.7) (drill 1) (layers "*.Cu" "*.Mask") (remove_unused_layers no) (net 61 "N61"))
  (pad "15" thru_hole circle (at 33.02 17.78 90) (size 1.7 1.7) (drill 1) (layers "*.Cu" "*.Mask") (remove_unused_layers no) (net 59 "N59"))
  (pad "16" thru_hole circle (at 30.48 17.78 90) (size 1.7 1.7) (drill 1) (layers "*.Cu" "*.Mask") (remove_unused_layers no) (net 58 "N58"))
  (pad "17" thru_hole circle (at 27.94 17.78 90) (size 1.7 1.7) (drill 1) (layers "*.Cu" "*.Mask") (remove_unused_layers no) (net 63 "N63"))
  (pad "18" thru_hole circle (at 25.4 17.78 90) (size 1.7 1.7) (drill 1) (layers "*.Cu" "*.Mask") (remove_unused_layers no) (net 16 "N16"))
  (pad "19" thru_hole circle (at 22.86 17.78 90) (size 1.7 1.7) (drill 1) (layers "*.Cu" "*.Mask") (remove_unused_layers no) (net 15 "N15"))
  (pad "20" thru_hole circle (at 20.32 17.78 90) (size 1.7 1.7) (drill 1) (layers "*.Cu" "*.Mask") (remove_unused_layers no) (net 11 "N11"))
  (pad "21" thru_hole circle (at 17.78 17.78 90) (size 1.7 1.7) (drill 1) (layers "*.Cu" "*.Mask") (remove_unused_layers no) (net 6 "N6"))
  (pad "22" thru_hole circle (at 15.24 17.78 90) (size 1.7 1.7) (drill 1) (layers "*.Cu" "*.Mask") (remove_unused_layers no) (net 10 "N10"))
  (pad "23" thru_hole circle (at 12.7 17.78 90) (size 1.7 1.7) (drill 1) (layers "*.Cu" "*.Mask") (remove_unused_layers no) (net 4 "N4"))
  (pad "24" thru_hole circle (at 10.16 17.78 90) (size 1.7 1.7) (drill 1) (layers "*.Cu" "*.Mask") (remove_unused_layers no) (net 3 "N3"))
  (pad "25" thru_hole circle (at 7.62 17.78 90) (size 1.7 1.7) (drill 1) (layers "*.Cu" "*.Mask") (remove_unused_layers no) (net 13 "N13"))
  (pad "26" thru_hole circle (at 5.08 17.78 90) (size 1.7 1.7) (drill 1) (layers "*.Cu" "*.Mask") (remove_unused_layers no) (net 74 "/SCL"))
  (pad "27" thru_hole circle (at 2.54 17.78 90) (size 1.7 1.7) (drill 1) (layers "*.Cu" "*.Mask") (remove_unused_layers no) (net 75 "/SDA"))
  (pad "28" thru_hole rect (at 0 17.78 90) (size 1.7 1.7) (drill 1) (layers "*.Cu" "*.Mask") (remove_unused_layers no) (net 76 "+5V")))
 (gr_line (start 83.5 108.5) (end 83.5 63.5) (stroke (width 0.05) (type default)) (layer "Edge.Cuts"))
 (gr_line (start 161 63.5) (end 206 63.5) (stroke (width 0.05) (type default)) (layer "Edge.Cuts"))
 (gr_line (start 161 141) (end 116 141) (stroke (width 0.05) (type default)) (layer "Edge.Cuts"))
 (gr_line (start 206 108.5) (end 161 108.5) (stroke (width 0.05) (type default)) (layer "Edge.Cuts"))
 (gr_line (start 116 108.5) (end 83.5 108.5) (stroke (width 0.05) (type default)) (layer "Edge.Cuts"))
 (gr_line (start 161 108.5) (end 161 141) (stroke (width 0.05) (type default)) (layer "Edge.Cuts"))
 (gr_line (start 206 63.5) (end 206 108.5) (stroke (width 0.05) (type default)) (layer "Edge.Cuts"))
 (gr_line (start 116 63.5) (end 116 31) (stroke (width 0.05) (type default)) (layer "Edge.Cuts"))
 (gr_line (start 116 31) (end 161 31) (stroke (width 0.05) (type default)) (layer "Edge.Cuts"))
 (gr_line (start 116 141) (end 116 108.5) (stroke (width 0.05) (type default)) (layer "Edge.Cuts"))
 (gr_line (start 83.5 63.5) (end 116 63.5) (stroke (width 0.05) (type default)) (layer "Edge.Cuts"))
 (gr_line (start 161 63.5) (end 161 31) (stroke (width 0.05) (type default)) (layer "Edge.Cuts"))
 (segment (start 203.5 89.08) (end 203.5 89.742) (width 0.2) (layer "F.Cu") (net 17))
 (segment (start 202.998 84) (end 203.5 84) (width 0.2) (layer "F.Cu") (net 75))
 (segment (start 199.002 76.962) (end 198.5 76.962) (width 0.2) (layer "F.Cu") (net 76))
 (segment (start 193.922 76.962) (end 193.42 76.962) (width 0.2) (layer "F.Cu") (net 74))
 (segment (start 107.27 98) (end 104.14 94.87) (width 0.2) (layer "B.Cu") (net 22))
 (segment (start 104.14 94.87) (end 104.14 94.742) (width 0.2) (layer "B.Cu") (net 22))
 (segment (start 113.291 94.26524) (end 112.61676 93.591) (width 0.2) (layer "F.Cu") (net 24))
 (segment (start 112.35 98) (end 113.291 97.059) (width 0.2) (layer "F.Cu") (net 24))
 (segment (start 110.371 93.591) (end 109.22 94.742) (width 0.2) (layer "F.Cu") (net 24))
 (segment (start 113.291 97.059) (end 113.291 94.26524) (width 0.2) (layer "F.Cu") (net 24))
 (segment (start 112.61676 93.591) (end 110.371 93.591) (width 0.2) (layer "F.Cu") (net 24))
 (segment (start 116.84 96.05) (end 116.84 94.742) (width 0.2) (layer "F.Cu") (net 25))
 (segment (start 114.89 98) (end 116.84 96.05) (width 0.2) (layer "F.Cu") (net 25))
 (segment (start 110.609 95.893) (end 111.76 94.742) (width 0.2) (layer "F.Cu") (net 18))
 (segment (start 99.217 95.893) (end 110.609 95.893) (width 0.2) (layer "F.Cu") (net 18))
 (segment (start 97.11 98) (end 99.217 95.893) (width 0.2) (layer "F.Cu") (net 18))
 (segment (start 115.034 93.19) (end 108.232 93.19) (width 0.2) (layer "F.Cu") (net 19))
 (segment (start 115.831 93.987) (end 115.034 93.19) (width 0.2) (layer "F.Cu") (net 19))
 (segment (start 108.232 93.19) (end 106.68 94.742) (width 0.2) (layer "F.Cu") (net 19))
 (segment (start 111.199 99.261) (end 111.252 99.314) (width 0.2) (layer "F.Cu") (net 19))
 (segment (start 109.95776 96.52) (end 111.199 97.76124) (width 0.2) (layer "F.Cu") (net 19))
 (segment (start 113.501 97.54876) (end 115.831 95.21876) (width 0.2) (layer "F.Cu") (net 19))
 (segment (start 112.776 99.314) (end 113.501 98.589) (width 0.2) (layer "F.Cu") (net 19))
 (segment (start 111.252 99.314) (end 112.776 99.314) (width 0.2) (layer "F.Cu") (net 19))
 (segment (start 111.199 97.76124) (end 111.199 99.261) (width 0.2) (layer "F.Cu") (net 19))
 (segment (start 99.65 98) (end 101.13 96.52) (width 0.2) (layer "F.Cu") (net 19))
 (segment (start 115.831 95.21876) (end 115.831 93.987) (width 0.2) (layer "F.Cu") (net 19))
 (segment (start 101.13 96.52) (end 109.95776 96.52) (width 0.2) (layer "F.Cu") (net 19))
 (segment (start 113.501 98.589) (end 113.501 97.54876) (width 0.2) (layer "F.Cu") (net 19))
 (segment (start 96.266 101.6) (end 92.964 98.298) (width 0.2) (layer "F.Cu") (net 23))
 (segment (start 92.964 98.298) (end 92.964 95.758) (width 0.2) (layer "F.Cu") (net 23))
 (segment (start 92.964 95.758) (end 93.98 94.742) (width 0.2) (layer "F.Cu") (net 23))
 (segment (start 109.81 98) (end 106.21 101.6) (width 0.2) (layer "F.Cu") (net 23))
 (segment (start 106.21 101.6) (end 96.266 101.6) (width 0.2) (layer "F.Cu") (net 23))
 (segment (start 96.3251 101.092) (end 101.638 101.092) (width 0.2) (layer "F.Cu") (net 21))
 (segment (start 95.511 81.033) (end 95.511 95.751) (width 0.2) (layer "F.Cu") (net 21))
 (segment (start 94.742 96.52) (end 94.742 99.5089) (width 0.2) (layer "F.Cu") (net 21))
 (segment (start 101.638 101.092) (end 104.73 98) (width 0.2) (layer "F.Cu") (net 21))
 (segment (start 91.44 76.962) (end 95.511 81.033) (width 0.2) (layer "F.Cu") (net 21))
 (segment (start 94.742 99.5089) (end 96.3251 101.092) (width 0.2) (layer "F.Cu") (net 21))
 (segment (start 95.511 95.751) (end 94.742 96.52) (width 0.2) (layer "F.Cu") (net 21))
 (segment (start 99.88955 100.30045) (end 96.49045 100.30045) (width 0.2) (layer "F.Cu") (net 20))
 (segment (start 98.051 95.497) (end 98.051 81.033) (width 0.2) (layer "F.Cu") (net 20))
 (segment (start 96.49045 100.30045) (end 95.369 99.179) (width 0.2) (layer "F.Cu") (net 20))
 (segment (start 95.369 97.439) (end 96.796 96.012) (width 0.2) (layer "F.Cu") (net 20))
 (segment (start 97.536 96.012) (end 98.051 95.497) (width 0.2) (layer "F.Cu") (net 20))
 (segment (start 95.369 99.179) (end 95.369 97.439) (width 0.2) (layer "F.Cu") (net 20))
 (segment (start 98.051 81.033) (end 93.98 76.962) (width 0.2) (layer "F.Cu") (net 20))
 (segment (start 102.19 98) (end 99.88955 100.30045) (width 0.2) (layer "F.Cu") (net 20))
 (segment (start 96.796 96.012) (end 97.536 96.012) (width 0.2) (layer "F.Cu") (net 20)))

